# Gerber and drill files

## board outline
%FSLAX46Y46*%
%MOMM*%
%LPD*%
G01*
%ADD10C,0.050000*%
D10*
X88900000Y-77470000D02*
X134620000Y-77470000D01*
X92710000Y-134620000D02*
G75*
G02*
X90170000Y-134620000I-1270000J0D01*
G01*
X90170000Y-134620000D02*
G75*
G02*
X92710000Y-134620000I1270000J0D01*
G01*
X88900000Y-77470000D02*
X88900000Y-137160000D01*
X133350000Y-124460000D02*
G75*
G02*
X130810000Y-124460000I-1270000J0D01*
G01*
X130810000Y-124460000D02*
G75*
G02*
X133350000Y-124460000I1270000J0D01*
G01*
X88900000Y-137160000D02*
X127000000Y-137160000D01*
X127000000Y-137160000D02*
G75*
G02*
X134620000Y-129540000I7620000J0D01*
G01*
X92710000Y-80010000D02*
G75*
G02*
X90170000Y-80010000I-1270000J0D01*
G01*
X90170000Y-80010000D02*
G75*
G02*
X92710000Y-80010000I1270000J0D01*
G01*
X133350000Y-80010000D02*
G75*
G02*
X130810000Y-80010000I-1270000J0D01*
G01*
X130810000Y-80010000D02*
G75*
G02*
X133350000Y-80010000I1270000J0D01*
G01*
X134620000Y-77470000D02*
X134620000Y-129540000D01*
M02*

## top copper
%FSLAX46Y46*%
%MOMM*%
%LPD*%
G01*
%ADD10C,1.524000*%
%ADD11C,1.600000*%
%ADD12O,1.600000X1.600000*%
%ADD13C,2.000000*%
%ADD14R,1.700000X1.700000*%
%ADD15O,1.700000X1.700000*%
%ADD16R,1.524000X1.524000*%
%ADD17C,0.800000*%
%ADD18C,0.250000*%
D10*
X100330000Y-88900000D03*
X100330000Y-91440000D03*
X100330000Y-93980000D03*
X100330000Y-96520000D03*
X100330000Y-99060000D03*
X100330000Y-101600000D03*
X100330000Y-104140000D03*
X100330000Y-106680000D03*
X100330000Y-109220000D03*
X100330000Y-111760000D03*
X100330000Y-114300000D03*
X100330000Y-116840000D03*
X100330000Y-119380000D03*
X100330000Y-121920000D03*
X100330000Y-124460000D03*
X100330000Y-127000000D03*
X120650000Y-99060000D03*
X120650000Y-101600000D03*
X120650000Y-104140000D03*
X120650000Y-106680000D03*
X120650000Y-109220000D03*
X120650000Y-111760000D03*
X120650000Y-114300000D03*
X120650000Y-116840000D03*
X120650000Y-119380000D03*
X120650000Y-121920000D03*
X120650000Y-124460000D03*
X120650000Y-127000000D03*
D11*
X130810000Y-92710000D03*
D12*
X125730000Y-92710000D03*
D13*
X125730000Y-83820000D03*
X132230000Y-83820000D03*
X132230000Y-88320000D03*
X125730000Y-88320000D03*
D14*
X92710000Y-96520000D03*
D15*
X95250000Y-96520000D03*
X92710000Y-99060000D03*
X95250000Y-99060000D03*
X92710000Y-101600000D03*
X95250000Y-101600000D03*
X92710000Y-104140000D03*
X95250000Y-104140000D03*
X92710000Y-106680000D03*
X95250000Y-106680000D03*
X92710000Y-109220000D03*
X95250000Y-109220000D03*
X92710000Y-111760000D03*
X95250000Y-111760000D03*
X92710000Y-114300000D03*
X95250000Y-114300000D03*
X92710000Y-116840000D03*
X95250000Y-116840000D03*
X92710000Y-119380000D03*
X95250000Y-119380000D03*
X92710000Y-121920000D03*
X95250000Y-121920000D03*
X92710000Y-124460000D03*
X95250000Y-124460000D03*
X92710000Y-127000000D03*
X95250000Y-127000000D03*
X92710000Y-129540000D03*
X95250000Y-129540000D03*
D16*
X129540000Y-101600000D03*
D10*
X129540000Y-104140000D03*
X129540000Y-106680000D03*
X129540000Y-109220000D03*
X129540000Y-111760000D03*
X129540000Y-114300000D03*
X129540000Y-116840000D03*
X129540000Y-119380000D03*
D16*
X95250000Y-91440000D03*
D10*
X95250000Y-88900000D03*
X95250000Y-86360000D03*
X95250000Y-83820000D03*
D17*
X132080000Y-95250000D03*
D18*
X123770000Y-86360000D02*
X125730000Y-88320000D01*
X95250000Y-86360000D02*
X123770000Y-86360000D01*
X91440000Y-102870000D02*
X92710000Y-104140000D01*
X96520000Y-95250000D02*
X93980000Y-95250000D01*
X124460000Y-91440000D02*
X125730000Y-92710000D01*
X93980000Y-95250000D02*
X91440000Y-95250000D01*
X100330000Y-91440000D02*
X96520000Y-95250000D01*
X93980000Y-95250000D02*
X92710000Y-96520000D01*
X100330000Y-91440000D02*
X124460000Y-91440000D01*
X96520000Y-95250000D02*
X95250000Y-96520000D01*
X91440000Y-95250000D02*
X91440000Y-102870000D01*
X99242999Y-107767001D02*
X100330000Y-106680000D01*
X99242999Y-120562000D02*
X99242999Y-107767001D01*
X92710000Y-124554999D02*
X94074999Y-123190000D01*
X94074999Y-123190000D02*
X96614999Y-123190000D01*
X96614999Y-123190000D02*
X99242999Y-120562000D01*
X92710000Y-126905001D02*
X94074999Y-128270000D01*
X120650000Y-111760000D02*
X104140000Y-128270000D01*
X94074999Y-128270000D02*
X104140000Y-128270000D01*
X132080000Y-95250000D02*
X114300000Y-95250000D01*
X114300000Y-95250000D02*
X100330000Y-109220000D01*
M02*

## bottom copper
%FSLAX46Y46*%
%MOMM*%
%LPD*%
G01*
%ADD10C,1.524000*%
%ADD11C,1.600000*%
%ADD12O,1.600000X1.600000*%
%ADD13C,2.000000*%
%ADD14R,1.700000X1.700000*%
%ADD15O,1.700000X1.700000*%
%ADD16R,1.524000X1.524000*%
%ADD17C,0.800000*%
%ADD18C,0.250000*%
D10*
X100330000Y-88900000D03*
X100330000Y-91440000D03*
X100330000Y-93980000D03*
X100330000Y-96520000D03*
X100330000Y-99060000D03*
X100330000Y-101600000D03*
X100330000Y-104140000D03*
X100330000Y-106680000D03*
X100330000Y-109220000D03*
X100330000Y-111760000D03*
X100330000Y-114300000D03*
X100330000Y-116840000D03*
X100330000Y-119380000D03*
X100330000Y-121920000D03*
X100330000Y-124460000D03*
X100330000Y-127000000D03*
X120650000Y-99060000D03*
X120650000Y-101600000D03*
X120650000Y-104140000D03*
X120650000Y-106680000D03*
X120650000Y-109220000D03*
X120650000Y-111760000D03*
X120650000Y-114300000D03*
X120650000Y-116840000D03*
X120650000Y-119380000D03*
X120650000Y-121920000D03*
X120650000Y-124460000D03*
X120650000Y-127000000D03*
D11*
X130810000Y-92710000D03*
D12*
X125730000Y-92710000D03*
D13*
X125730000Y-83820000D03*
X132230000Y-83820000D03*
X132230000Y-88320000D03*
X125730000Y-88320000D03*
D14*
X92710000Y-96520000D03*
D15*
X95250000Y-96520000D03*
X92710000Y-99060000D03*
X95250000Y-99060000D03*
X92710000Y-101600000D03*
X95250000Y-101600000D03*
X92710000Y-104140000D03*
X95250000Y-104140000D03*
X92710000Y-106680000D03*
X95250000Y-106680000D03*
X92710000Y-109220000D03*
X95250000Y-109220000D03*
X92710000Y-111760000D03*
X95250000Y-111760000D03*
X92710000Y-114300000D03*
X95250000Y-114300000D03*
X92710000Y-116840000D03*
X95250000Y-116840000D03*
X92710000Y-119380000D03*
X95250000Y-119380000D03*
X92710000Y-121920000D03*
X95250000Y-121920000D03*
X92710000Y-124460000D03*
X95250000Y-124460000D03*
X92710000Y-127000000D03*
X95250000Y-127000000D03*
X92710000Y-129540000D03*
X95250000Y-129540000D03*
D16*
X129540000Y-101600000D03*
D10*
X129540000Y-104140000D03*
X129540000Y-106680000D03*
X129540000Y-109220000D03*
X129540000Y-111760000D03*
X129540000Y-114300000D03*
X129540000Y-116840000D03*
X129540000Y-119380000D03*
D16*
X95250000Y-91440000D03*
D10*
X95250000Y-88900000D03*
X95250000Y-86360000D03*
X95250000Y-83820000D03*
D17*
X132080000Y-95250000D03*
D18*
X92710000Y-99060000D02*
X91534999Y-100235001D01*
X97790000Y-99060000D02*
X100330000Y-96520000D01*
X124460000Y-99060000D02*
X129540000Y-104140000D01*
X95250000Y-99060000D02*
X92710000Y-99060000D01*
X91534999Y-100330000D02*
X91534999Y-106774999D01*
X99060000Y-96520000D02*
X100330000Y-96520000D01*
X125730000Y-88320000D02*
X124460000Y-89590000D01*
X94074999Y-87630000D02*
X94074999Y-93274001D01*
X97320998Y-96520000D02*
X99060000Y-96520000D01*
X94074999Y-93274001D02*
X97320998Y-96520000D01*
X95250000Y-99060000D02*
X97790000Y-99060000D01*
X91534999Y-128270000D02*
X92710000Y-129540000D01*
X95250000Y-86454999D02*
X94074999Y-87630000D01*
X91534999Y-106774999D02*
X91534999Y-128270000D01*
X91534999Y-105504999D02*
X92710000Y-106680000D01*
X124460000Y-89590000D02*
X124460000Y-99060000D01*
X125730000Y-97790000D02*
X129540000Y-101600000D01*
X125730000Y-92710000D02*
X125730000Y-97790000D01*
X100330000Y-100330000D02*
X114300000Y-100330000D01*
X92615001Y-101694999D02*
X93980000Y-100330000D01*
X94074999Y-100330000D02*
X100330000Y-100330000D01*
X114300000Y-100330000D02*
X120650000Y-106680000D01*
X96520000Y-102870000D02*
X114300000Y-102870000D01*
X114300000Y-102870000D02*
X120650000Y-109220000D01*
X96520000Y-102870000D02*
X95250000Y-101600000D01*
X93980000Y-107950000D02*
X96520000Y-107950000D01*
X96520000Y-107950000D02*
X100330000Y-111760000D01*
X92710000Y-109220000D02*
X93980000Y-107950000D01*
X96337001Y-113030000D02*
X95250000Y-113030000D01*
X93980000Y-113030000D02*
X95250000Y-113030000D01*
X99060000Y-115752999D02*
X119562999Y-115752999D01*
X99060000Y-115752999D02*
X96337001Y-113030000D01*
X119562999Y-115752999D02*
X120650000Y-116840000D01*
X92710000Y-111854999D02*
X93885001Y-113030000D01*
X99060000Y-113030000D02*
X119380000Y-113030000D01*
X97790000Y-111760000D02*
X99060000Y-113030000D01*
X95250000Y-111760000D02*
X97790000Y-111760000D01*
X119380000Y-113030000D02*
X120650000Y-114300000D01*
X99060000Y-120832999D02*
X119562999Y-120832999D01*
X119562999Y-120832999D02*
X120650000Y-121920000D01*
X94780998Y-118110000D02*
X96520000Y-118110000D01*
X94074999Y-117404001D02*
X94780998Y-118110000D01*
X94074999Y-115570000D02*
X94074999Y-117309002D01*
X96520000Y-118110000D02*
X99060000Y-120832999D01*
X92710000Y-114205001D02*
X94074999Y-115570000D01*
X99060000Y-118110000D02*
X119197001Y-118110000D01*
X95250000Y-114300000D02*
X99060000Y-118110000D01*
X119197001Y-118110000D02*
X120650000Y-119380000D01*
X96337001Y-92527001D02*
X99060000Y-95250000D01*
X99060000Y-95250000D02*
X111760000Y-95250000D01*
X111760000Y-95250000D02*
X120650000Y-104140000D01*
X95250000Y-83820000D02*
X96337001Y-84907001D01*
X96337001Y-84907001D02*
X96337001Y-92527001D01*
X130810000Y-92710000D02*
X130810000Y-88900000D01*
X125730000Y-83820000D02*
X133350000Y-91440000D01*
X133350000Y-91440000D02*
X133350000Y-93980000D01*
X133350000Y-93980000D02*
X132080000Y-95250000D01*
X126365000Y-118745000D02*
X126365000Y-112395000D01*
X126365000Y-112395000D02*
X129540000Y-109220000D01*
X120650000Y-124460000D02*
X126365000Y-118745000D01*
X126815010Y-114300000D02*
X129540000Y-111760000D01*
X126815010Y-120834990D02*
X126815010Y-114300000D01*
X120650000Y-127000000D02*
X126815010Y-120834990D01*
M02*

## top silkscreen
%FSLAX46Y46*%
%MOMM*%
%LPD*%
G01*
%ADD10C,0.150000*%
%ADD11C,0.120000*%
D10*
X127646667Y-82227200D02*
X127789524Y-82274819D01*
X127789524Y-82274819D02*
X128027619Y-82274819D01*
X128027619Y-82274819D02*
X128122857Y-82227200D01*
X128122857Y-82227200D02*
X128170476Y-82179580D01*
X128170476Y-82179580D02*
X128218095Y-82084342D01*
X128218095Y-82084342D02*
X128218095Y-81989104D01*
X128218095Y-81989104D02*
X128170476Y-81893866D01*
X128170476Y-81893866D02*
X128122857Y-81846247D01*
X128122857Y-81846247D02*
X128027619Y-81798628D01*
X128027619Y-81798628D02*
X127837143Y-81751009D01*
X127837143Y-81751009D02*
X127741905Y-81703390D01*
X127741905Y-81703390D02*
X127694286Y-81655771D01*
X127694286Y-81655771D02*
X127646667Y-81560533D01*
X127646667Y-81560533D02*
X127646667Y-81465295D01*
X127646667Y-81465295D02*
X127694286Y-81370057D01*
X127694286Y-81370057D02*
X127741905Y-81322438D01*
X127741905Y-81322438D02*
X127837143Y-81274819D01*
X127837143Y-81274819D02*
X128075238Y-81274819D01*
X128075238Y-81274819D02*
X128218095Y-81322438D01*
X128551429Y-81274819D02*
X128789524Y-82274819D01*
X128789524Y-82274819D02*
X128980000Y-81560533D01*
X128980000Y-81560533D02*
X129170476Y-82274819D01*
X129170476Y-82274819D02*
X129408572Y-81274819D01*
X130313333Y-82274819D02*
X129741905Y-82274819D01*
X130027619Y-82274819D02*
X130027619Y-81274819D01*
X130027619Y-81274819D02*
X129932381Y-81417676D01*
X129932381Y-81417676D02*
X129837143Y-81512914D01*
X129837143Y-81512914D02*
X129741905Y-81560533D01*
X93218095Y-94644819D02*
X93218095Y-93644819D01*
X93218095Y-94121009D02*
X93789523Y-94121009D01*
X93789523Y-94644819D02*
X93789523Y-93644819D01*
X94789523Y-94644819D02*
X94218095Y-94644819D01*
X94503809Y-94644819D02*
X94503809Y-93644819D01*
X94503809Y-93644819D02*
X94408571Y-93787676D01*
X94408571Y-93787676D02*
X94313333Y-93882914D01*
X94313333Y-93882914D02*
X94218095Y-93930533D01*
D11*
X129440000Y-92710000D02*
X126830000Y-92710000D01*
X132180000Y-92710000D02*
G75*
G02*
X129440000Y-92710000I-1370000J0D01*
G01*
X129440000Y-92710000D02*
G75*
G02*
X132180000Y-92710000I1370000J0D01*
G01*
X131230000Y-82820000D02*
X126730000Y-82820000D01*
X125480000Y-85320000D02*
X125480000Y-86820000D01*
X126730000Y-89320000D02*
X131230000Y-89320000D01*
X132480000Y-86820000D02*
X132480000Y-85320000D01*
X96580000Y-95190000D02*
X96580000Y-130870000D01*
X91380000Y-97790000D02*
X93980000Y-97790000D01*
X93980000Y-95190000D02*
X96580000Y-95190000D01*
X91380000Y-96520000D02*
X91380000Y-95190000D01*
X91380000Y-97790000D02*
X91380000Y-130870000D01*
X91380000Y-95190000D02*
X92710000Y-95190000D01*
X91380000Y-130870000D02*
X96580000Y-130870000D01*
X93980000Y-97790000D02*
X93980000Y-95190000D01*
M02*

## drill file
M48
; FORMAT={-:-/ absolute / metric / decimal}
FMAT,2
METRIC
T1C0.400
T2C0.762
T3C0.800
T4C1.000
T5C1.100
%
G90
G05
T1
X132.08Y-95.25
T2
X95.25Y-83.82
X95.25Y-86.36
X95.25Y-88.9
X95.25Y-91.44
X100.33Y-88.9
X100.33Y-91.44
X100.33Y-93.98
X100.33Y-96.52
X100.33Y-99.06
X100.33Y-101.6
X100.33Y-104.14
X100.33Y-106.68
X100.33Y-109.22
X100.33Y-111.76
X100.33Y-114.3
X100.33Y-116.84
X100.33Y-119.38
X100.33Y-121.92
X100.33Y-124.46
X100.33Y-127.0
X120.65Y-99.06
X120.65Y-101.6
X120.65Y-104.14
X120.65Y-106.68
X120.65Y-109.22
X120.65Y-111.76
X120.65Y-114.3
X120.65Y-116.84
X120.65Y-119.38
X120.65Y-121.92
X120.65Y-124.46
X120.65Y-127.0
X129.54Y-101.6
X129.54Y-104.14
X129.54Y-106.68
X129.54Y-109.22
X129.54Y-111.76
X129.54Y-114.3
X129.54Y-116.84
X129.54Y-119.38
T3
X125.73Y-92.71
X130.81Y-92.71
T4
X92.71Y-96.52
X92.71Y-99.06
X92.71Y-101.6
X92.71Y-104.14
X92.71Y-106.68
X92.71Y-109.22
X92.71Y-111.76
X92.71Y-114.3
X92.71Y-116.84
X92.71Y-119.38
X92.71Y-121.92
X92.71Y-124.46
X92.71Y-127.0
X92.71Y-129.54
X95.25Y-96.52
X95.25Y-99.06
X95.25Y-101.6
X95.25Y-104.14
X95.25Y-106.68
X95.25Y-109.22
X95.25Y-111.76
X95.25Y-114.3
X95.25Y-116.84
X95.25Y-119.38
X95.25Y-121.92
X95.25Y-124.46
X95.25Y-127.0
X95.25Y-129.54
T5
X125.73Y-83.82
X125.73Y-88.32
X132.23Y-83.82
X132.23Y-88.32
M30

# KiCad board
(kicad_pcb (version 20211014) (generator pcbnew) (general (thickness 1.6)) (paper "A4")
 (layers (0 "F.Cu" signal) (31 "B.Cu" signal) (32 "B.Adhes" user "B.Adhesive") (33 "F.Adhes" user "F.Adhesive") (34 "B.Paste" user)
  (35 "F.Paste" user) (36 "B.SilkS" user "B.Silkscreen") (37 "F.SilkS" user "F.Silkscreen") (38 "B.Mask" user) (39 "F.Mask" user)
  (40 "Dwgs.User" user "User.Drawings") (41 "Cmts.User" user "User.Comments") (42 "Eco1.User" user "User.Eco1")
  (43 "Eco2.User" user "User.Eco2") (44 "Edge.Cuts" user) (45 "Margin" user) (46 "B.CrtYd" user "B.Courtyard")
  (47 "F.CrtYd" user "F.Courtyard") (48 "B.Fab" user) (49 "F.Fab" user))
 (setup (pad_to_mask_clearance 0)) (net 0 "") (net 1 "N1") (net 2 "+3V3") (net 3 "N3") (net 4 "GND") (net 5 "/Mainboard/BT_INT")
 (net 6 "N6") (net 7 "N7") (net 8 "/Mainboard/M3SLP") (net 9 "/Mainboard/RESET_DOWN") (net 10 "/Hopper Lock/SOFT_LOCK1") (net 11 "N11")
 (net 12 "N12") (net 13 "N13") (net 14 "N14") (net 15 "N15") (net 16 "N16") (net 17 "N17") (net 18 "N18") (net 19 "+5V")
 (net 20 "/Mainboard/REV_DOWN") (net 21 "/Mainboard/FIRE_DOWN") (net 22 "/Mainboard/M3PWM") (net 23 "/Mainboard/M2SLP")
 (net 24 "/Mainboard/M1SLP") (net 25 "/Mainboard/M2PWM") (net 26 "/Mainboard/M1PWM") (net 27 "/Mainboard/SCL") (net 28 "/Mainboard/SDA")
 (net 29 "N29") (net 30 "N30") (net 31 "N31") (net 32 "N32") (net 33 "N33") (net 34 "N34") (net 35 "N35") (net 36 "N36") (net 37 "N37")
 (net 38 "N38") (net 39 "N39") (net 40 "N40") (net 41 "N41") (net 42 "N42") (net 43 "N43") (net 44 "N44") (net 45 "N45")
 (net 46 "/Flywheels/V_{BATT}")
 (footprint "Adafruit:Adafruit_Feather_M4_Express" (layer "F.Cu") (at 110.49 107.95)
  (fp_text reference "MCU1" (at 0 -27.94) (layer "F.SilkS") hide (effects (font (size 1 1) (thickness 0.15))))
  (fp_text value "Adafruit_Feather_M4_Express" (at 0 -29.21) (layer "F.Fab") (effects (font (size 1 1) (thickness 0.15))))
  (pad "1" thru_hole circle locked (at -10.16 -19.05) (size 1.524 1.524) (drill 0.762) (layers *.Cu *.Mask) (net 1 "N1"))
  (pad "2" thru_hole circle locked (at -10.16 -16.51) (size 1.524 1.524) (drill 0.762) (layers *.Cu *.Mask) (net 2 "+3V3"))
  (pad "3" thru_hole circle locked (at -10.16 -13.97) (size 1.524 1.524) (drill 0.762) (layers *.Cu *.Mask) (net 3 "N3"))
  (pad "4" thru_hole circle locked (at -10.16 -11.43) (size 1.524 1.524) (drill 0.762) (layers *.Cu *.Mask) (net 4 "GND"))
  (pad "5" thru_hole circle locked (at -10.16 -8.89) (size 1.524 1.524) (drill 0.762) (layers *.Cu *.Mask) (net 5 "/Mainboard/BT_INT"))
  (pad "6" thru_hole circle locked (at -10.16 -6.35) (size 1.524 1.524) (drill 0.762) (layers *.Cu *.Mask) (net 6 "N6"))
  (pad "7" thru_hole circle locked (at -10.16 -3.81) (size 1.524 1.524) (drill 0.762) (layers *.Cu *.Mask) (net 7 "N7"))
  (pad "8" thru_hole circle locked (at -10.16 -1.27) (size 1.524 1.524) (drill 0.762) (layers *.Cu *.Mask) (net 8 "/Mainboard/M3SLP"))
  (pad "9" thru_hole circle locked (at -10.16 1.27) (size 1.524 1.524) (drill 0.762) (layers *.Cu *.Mask) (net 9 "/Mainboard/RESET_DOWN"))
  (pad "10" thru_hole circle locked (at -10.16 3.81) (size 1.524 1.524) (drill 0.762) (layers *.Cu *.Mask)
   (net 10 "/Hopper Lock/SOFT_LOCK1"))
  (pad "11" thru_hole circle locked (at -10.16 6.35) (size 1.524 1.524) (drill 0.762) (layers *.Cu *.Mask) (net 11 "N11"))
  (pad "12" thru_hole circle locked (at -10.16 8.89) (size 1.524 1.524) (drill 0.762) (layers *.Cu *.Mask) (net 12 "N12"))
  (pad "13" thru_hole circle locked (at -10.16 11.43) (size 1.524 1.524) (drill 0.762) (layers *.Cu *.Mask) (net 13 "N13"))
  (pad "14" thru_hole circle locked (at -10.16 13.97) (size 1.524 1.524) (drill 0.762) (layers *.Cu *.Mask) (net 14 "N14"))
  (pad "15" thru_hole circle locked (at -10.16 16.51) (size 1.524 1.524) (drill 0.762) (layers *.Cu *.Mask) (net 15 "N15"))
  (pad "16" thru_hole circle locked (at -10.16 19.05) (size 1.524 1.524) (drill 0.762) (layers *.Cu *.Mask) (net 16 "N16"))
  (pad "17" thru_hole circle locked (at 10.16 -8.89) (size 1.524 1.524) (drill 0.762) (layers *.Cu *.Mask) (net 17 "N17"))
  (pad "18" thru_hole circle locked (at 10.16 -6.35) (size 1.524 1.524) (drill 0.762) (layers *.Cu *.Mask) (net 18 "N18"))
  (pad "19" thru_hole circle locked (at 10.16 -3.81) (size 1.524 1.524) (drill 0.762) (layers *.Cu *.Mask) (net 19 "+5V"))
  (pad "20" thru_hole circle locked (at 10.16 -1.27) (size 1.524 1.524) (drill 0.762) (layers *.Cu *.Mask) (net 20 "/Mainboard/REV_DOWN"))
  (pad "21" thru_hole circle locked (at 10.16 1.27) (size 1.524 1.524) (drill 0.762) (layers *.Cu *.Mask) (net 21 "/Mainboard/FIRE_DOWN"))
  (pad "22" thru_hole circle locked (at 10.16 3.81) (size 1.524 1.524) (drill 0.762) (layers *.Cu *.Mask) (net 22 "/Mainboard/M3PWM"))
  (pad "23" thru_hole circle locked (at 10.16 6.35) (size 1.524 1.524) (drill 0.762) (layers *.Cu *.Mask) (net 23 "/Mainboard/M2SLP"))
  (pad "24" thru_hole circle locked (at 10.16 8.89) (size 1.524 1.524) (drill 0.762) (layers *.Cu *.Mask) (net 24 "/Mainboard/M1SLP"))
  (pad "25" thru_hole circle locked (at 10.16 11.43) (size 1.524 1.524) (drill 0.762) (layers *.Cu *.Mask) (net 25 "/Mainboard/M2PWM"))
  (pad "26" thru_hole circle locked (at 10.16 13.97) (size 1.524 1.524) (drill 0.762) (layers *.Cu *.Mask) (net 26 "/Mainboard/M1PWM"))
  (pad "27" thru_hole circle locked (at 10.16 16.51) (size 1.524 1.524) (drill 0.762) (layers *.Cu *.Mask) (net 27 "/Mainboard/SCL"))
  (pad "28" thru_hole circle locked (at 10.16 19.05) (size 1.524 1.524) (drill 0.762) (layers *.Cu *.Mask) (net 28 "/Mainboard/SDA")))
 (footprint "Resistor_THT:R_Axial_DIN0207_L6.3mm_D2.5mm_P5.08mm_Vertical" (layer "F.Cu") (at 130.81 92.71 180)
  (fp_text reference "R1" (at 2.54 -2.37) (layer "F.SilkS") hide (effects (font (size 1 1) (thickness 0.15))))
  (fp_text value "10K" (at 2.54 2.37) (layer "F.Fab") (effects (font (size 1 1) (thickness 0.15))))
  (fp_line (start 1.37 0) (end 3.98 0) (layer "F.SilkS") (width 0.12))
  (fp_circle (center 0 0) (end 1.37 0) (layer "F.SilkS") (width 0.12) (fill none))
  (pad "1" thru_hole circle locked (at 0 0 180) (size 1.6 1.6) (drill 0.8) (layers *.Cu *.Mask) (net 9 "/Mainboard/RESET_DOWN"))
  (pad "2" thru_hole oval locked (at 5.08 0 180) (size 1.6 1.6) (drill 0.8) (layers *.Cu *.Mask) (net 2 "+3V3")))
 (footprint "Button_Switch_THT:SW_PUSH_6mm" (layer "F.Cu") (at 125.73 83.82)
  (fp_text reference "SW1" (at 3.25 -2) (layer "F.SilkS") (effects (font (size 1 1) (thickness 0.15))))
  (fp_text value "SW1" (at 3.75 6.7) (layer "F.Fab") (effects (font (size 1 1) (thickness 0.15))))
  (fp_line (start 5.5 -1) (end 1 -1) (layer "F.SilkS") (width 0.12))
  (fp_line (start -0.25 1.5) (end -0.25 3) (layer "F.SilkS") (width 0.12))
  (fp_line (start 1 5.5) (end 5.5 5.5) (layer "F.SilkS") (width 0.12))
  (fp_line (start 6.75 3) (end 6.75 1.5) (layer "F.SilkS") (width 0.12))
  (pad "1" thru_hole circle locked (at 0 0 90) (size 2 2) (drill 1.1) (layers *.Cu *.Mask) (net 9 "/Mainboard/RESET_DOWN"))
  (pad "1" thru_hole circle locked (at 6.5 0 90) (size 2 2) (drill 1.1) (layers *.Cu *.Mask) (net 9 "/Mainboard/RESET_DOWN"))
  (pad "2" thru_hole circle locked (at 6.5 4.5 90) (size 2 2) (drill 1.1) (layers *.Cu *.Mask) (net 4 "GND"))
  (pad "2" thru_hole circle locked (at 0 4.5 90) (size 2 2) (drill 1.1) (layers *.Cu *.Mask) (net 4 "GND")))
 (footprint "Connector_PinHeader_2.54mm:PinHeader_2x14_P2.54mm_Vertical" (layer "F.Cu") (at 92.71 96.52)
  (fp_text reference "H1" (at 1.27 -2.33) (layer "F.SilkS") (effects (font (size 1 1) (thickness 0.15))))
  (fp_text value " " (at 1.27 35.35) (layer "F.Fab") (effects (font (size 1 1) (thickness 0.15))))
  (fp_line (start 3.87 -1.33) (end 3.87 34.35) (layer "F.SilkS") (width 0.12))
  (fp_line (start -1.33 1.27) (end 1.27 1.27) (layer "F.SilkS") (width 0.12))
  (fp_line (start 1.27 -1.33) (end 3.87 -1.33) (layer "F.SilkS") (width 0.12))
  (fp_line (start -1.33 0) (end -1.33 -1.33) (layer "F.SilkS") (width 0.12))
  (fp_line (start -1.33 1.27) (end -1.33 34.35) (layer "F.SilkS") (width 0.12))
  (fp_line (start -1.33 -1.33) (end 0 -1.33) (layer "F.SilkS") (width 0.12))
  (fp_line (start -1.33 34.35) (end 3.87 34.35) (layer "F.SilkS") (width 0.12))
  (fp_line (start 1.27 1.27) (end 1.27 -1.33) (layer "F.SilkS") (width 0.12))
  (pad "1" thru_hole rect locked (at 0 0) (size 1.7 1.7) (drill 1) (layers *.Cu *.Mask) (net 2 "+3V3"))
  (pad "2" thru_hole oval locked (at 2.54 0) (size 1.7 1.7) (drill 1) (layers *.Cu *.Mask) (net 2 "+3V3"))
  (pad "3" thru_hole oval locked (at 0 2.54) (size 1.7 1.7) (drill 1) (layers *.Cu *.Mask) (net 4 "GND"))
  (pad "4" thru_hole oval locked (at 2.54 2.54) (size 1.7 1.7) (drill 1) (layers *.Cu *.Mask) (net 4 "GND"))
  (pad "5" thru_hole oval locked (at 0 5.08) (size 1.7 1.7) (drill 1) (layers *.Cu *.Mask) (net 20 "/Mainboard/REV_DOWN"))
  (pad "6" thru_hole oval locked (at 2.54 5.08) (size 1.7 1.7) (drill 1) (layers *.Cu *.Mask) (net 21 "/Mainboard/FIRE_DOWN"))
  (pad "7" thru_hole oval locked (at 0 7.62) (size 1.7 1.7) (drill 1) (layers *.Cu *.Mask) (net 2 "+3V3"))
  (pad "8" thru_hole oval locked (at 2.54 7.62) (size 1.7 1.7) (drill 1) (layers *.Cu *.Mask) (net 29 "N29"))
  (pad "9" thru_hole oval locked (at 0 10.16) (size 1.7 1.7) (drill 1) (layers *.Cu *.Mask) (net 4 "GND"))
  (pad "10" thru_hole oval locked (at 2.54 10.16) (size 1.7 1.7) (drill 1) (layers *.Cu *.Mask) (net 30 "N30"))
  (pad "11" thru_hole oval locked (at 0 12.7) (size 1.7 1.7) (drill 1) (layers *.Cu *.Mask) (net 10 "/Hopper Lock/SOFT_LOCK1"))
  (pad "12" thru_hole oval locked (at 2.54 12.7) (size 1.7 1.7) (drill 1) (layers *.Cu *.Mask) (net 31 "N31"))
  (pad "13" thru_hole oval locked (at 0 15.24) (size 1.7 1.7) (drill 1) (layers *.Cu *.Mask) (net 24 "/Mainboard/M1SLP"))
  (pad "14" thru_hole oval locked (at 2.54 15.24) (size 1.7 1.7) (drill 1) (layers *.Cu *.Mask) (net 23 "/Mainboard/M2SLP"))
  (pad "15" thru_hole oval locked (at 0 17.78) (size 1.7 1.7) (drill 1) (layers *.Cu *.Mask) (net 26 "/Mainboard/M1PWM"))
  (pad "16" thru_hole oval locked (at 2.54 17.78) (size 1.7 1.7) (drill 1) (layers *.Cu *.Mask) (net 25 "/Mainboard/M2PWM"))
  (pad "17" thru_hole oval locked (at 0 20.32) (size 1.7 1.7) (drill 1) (layers *.Cu *.Mask) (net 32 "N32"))
  (pad "18" thru_hole oval locked (at 2.54 20.32) (size 1.7 1.7) (drill 1) (layers *.Cu *.Mask) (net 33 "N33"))
  (pad "19" thru_hole oval locked (at 0 22.86) (size 1.7 1.7) (drill 1) (layers *.Cu *.Mask) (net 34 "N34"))
  (pad "20" thru_hole oval locked (at 2.54 22.86) (size 1.7 1.7) (drill 1) (layers *.Cu *.Mask) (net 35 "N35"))
  (pad "21" thru_hole oval locked (at 0 25.4) (size 1.7 1.7) (drill 1) (layers *.Cu *.Mask) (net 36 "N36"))
  (pad "22" thru_hole oval locked (at 2.54 25.4) (size 1.7 1.7) (drill 1) (layers *.Cu *.Mask) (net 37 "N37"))
  (pad "23" thru_hole oval locked (at 0 27.94) (size 1.7 1.7) (drill 1) (layers *.Cu *.Mask) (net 8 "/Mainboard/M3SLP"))
  (pad "24" thru_hole oval locked (at 2.54 27.94) (size 1.7 1.7) (drill 1) (layers *.Cu *.Mask) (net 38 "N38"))
  (pad "25" thru_hole oval locked (at 0 30.48) (size 1.7 1.7) (drill 1) (layers *.Cu *.Mask) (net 22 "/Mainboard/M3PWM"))
  (pad "26" thru_hole oval locked (at 2.54 30.48) (size 1.7 1.7) (drill 1) (layers *.Cu *.Mask) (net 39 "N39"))
  (pad "27" thru_hole oval locked (at 0 33.02) (size 1.7 1.7) (drill 1) (layers *.Cu *.Mask) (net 4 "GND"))
  (pad "28" thru_hole oval locked (at 2.54 33.02) (size 1.7 1.7) (drill 1) (layers *.Cu *.Mask) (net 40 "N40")))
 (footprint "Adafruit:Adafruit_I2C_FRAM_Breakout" (layer "B.Cu") (at 124.46 110.49 -90)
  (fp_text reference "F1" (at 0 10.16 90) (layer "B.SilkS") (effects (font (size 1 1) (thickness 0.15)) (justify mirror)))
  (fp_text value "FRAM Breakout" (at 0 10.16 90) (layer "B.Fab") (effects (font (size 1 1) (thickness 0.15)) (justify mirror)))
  (pad "1" thru_hole rect locked (at -8.89 -5.08 270) (size 1.524 1.524) (drill 0.762) (layers *.Cu *.Mask) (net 2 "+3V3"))
  (pad "2" thru_hole circle locked (at -6.35 -5.08 270) (size 1.524 1.524) (drill 0.762) (layers *.Cu *.Mask) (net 4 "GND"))
  (pad "3" thru_hole circle locked (at -3.81 -5.08 270) (size 1.524 1.524) (drill 0.762) (layers *.Cu *.Mask) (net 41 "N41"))
  (pad "4" thru_hole circle locked (at -1.27 -5.08 270) (size 1.524 1.524) (drill 0.762) (layers *.Cu *.Mask) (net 27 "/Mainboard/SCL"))
  (pad "5" thru_hole circle locked (at 1.27 -5.08 270) (size 1.524 1.524) (drill 0.762) (layers *.Cu *.Mask) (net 28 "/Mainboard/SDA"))
  (pad "6" thru_hole circle locked (at 3.81 -5.08 270) (size 1.524 1.524) (drill 0.762) (layers *.Cu *.Mask) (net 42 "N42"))
  (pad "7" thru_hole circle locked (at 6.35 -5.08 270) (size 1.524 1.524) (drill 0.762) (layers *.Cu *.Mask) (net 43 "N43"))
  (pad "8" thru_hole circle locked (at 8.89 -5.08 270) (size 1.524 1.524) (drill 0.762) (layers *.Cu *.Mask) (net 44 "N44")))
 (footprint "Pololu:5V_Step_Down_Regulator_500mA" (layer "B.Cu") (at 100.33 87.63 90)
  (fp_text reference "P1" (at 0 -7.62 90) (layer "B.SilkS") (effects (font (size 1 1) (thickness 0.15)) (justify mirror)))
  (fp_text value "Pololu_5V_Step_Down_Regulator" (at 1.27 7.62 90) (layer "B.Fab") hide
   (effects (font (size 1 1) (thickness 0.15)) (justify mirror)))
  (pad "1" thru_hole rect locked (at -3.81 -5.08 90) (size 1.524 1.524) (drill 0.762) (layers *.Cu *.Mask) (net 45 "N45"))
  (pad "2" thru_hole circle locked (at -1.27 -5.08 90) (size 1.524 1.524) (drill 0.762) (layers *.Cu *.Mask) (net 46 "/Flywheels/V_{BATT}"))
  (pad "3" thru_hole circle locked (at 1.27 -5.08 90) (size 1.524 1.524) (drill 0.762) (layers *.Cu *.Mask) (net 4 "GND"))
  (pad "4" thru_hole circle locked (at 3.81 -5.08 90) (size 1.524 1.524) (drill 0.762) (layers *.Cu *.Mask) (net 19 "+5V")))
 (gr_line (start 88.9 77.47) (end 134.62 77.47) (layer "Edge.Cuts") (width 0.05))
 (gr_circle (center 91.44 134.62) (end 91.44 135.89) (layer "Edge.Cuts") (width 0.05) (fill none))
 (gr_line (start 88.9 77.47) (end 88.9 137.16) (layer "Edge.Cuts") (width 0.05))
 (gr_circle (center 132.08 124.46) (end 133.35 124.46) (layer "Edge.Cuts") (width 0.05) (fill none))
 (gr_line (start 88.9 137.16) (end 127 137.16) (layer "Edge.Cuts") (width 0.05))
 (gr_arc (start 127 137.16) (mid 129.231846 131.771846) (end 134.62 129.54) (layer "Edge.Cuts") (width 0.05))
 (gr_circle (center 91.44 80.01) (end 90.17 80.01) (layer "Edge.Cuts") (width 0.05) (fill none))
 (gr_circle (center 132.08 80.01) (end 133.35 80.01) (layer "Edge.Cuts") (width 0.05) (fill none))
 (gr_line (start 134.62 77.47) (end 134.62 129.54) (layer "Edge.Cuts") (width 0.05))
 (segment (start 123.77 86.36) (end 125.73 88.32) (width 0.25) (layer "F.Cu") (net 4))
 (segment (start 95.25 86.36) (end 123.77 86.36) (width 0.25) (layer "F.Cu") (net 4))
 (segment (start 92.71 99.06) (end 91.534999 100.235001) (width 0.25) (layer "B.Cu") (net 4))
 (segment (start 97.79 99.06) (end 100.33 96.52) (width 0.25) (layer "B.Cu") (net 4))
 (segment (start 124.46 99.06) (end 129.54 104.14) (width 0.25) (layer "B.Cu") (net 4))
 (segment (start 95.25 99.06) (end 92.71 99.06) (width 0.25) (layer "B.Cu") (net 4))
 (segment (start 91.534999 100.33) (end 91.534999 106.774999) (width 0.25) (layer "B.Cu") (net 4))
 (segment (start 99.06 96.52) (end 100.33 96.52) (width 0.25) (layer "B.Cu") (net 4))
 (segment (start 125.73 88.32) (end 124.46 89.59) (width 0.25) (layer "B.Cu") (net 4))
 (segment (start 94.074999 87.63) (end 94.074999 93.274001) (width 0.25) (layer "B.Cu") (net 4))
 (segment (start 97.320998 96.52) (end 99.06 96.52) (width 0.25) (layer "B.Cu") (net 4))
 (segment (start 94.074999 93.274001) (end 97.320998 96.52) (width 0.25) (layer "B.Cu") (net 4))
 (segment (start 95.25 99.06) (end 97.79 99.06) (width 0.25) (layer "B.Cu") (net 4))
 (segment (start 91.534999 128.27) (end 92.71 129.54) (width 0.25) (layer "B.Cu") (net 4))
 (segment (start 95.25 86.454999) (end 94.074999 87.63) (width 0.25) (layer "B.Cu") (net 4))
 (segment (start 91.534999 106.774999) (end 91.534999 128.27) (width 0.25) (layer "B.Cu") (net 4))
 (segment (start 91.534999 105.504999) (end 92.71 106.68) (width 0.25) (layer "B.Cu") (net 4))
 (segment (start 124.46 89.59) (end 124.46 99.06) (width 0.25) (layer "B.Cu") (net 4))
 (segment (start 91.44 102.87) (end 92.71 104.14) (width 0.25) (layer "F.Cu") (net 2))
 (segment (start 96.52 95.25) (end 93.98 95.25) (width 0.25) (layer "F.Cu") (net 2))
 (segment (start 124.46 91.44) (end 125.73 92.71) (width 0.25) (layer "F.Cu") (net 2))
 (segment (start 93.98 95.25) (end 91.44 95.25) (width 0.25) (layer "F.Cu") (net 2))
 (segment (start 100.33 91.44) (end 96.52 95.25) (width 0.25) (layer "F.Cu") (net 2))
 (segment (start 93.98 95.25) (end 92.71 96.52) (width 0.25) (layer "F.Cu") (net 2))
 (segment (start 100.33 91.44) (end 124.46 91.44) (width 0.25) (layer "F.Cu") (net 2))
 (segment (start 96.52 95.25) (end 95.25 96.52) (width 0.25) (layer "F.Cu") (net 2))
 (segment (start 91.44 95.25) (end 91.44 102.87) (width 0.25) (layer "F.Cu") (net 2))
 (segment (start 125.73 97.79) (end 129.54 101.6) (width 0.25) (layer "B.Cu") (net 2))
 (segment (start 125.73 92.71) (end 125.73 97.79) (width 0.25) (layer "B.Cu") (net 2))
 (segment (start 100.33 100.33) (end 114.3 100.33) (width 0.25) (layer "B.Cu") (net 20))
 (segment (start 92.615001 101.694999) (end 93.98 100.33) (width 0.25) (layer "B.Cu") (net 20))
 (segment (start 94.074999 100.33) (end 100.33 100.33) (width 0.25) (layer "B.Cu") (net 20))
 (segment (start 114.3 100.33) (end 120.65 106.68) (width 0.25) (layer "B.Cu") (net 20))
 (segment (start 96.52 102.87) (end 114.3 102.87) (width 0.25) (layer "B.Cu") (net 21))
 (segment (start 114.3 102.87) (end 120.65 109.22) (width 0.25) (layer "B.Cu") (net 21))
 (segment (start 96.52 102.87) (end 95.25 101.6) (width 0.25) (layer "B.Cu") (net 21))
 (segment (start 93.98 107.95) (end 96.52 107.95) (width 0.25) (layer "B.Cu") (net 10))
 (segment (start 96.52 107.95) (end 100.33 111.76) (width 0.25) (layer "B.Cu") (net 10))
 (segment (start 92.71 109.22) (end 93.98 107.95) (width 0.25) (layer "B.Cu") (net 10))
 (segment (start 96.337001 113.03) (end 95.25 113.03) (width 0.25) (layer "B.Cu") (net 24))
 (segment (start 93.98 113.03) (end 95.25 113.03) (width 0.25) (layer "B.Cu") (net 24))
 (segment (start 99.06 115.752999) (end 119.562999 115.752999) (width 0.25) (layer "B.Cu") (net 24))
 (segment (start 99.06 115.752999) (end 96.337001 113.03) (width 0.25) (layer "B.Cu") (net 24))
 (segment (start 119.562999 115.752999) (end 120.65 116.84) (width 0.25) (layer "B.Cu") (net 24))
 (segment (start 92.71 111.854999) (end 93.885001 113.03) (width 0.25) (layer "B.Cu") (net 24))
 (segment (start 99.06 113.03) (end 119.38 113.03) (width 0.25) (layer "B.Cu") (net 23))
 (segment (start 97.79 111.76) (end 99.06 113.03) (width 0.25) (layer "B.Cu") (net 23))
 (segment (start 95.25 111.76) (end 97.79 111.76) (width 0.25) (layer "B.Cu") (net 23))
 (segment (start 119.38 113.03) (end 120.65 114.3) (width 0.25) (layer "B.Cu") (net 23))
 (segment (start 99.06 120.832999) (end 119.562999 120.832999) (width 0.25) (layer "B.Cu") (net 26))
 (segment (start 119.562999 120.832999) (end 120.65 121.92) (width 0.25) (layer "B.Cu") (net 26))
 (segment (start 94.780998 118.11) (end 96.52 118.11) (width 0.25) (layer "B.Cu") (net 26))
 (segment (start 94.074999 117.404001) (end 94.780998 118.11) (width 0.25) (layer "B.Cu") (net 26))
 (segment (start 94.074999 115.57) (end 94.074999 117.309002) (width 0.25) (layer "B.Cu") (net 26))
 (segment (start 96.52 118.11) (end 99.06 120.832999) (width 0.25) (layer "B.Cu") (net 26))
 (segment (start 92.71 114.205001) (end 94.074999 115.57) (width 0.25) (layer "B.Cu") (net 26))
 (segment (start 99.06 118.11) (end 119.197001 118.11) (width 0.25) (layer "B.Cu") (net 25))
 (segment (start 95.25 114.3) (end 99.06 118.11) (width 0.25) (layer "B.Cu") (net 25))
 (segment (start 119.197001 118.11) (end 120.65 119.38) (width 0.25) (layer "B.Cu") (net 25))
 (segment (start 99.242999 107.767001) (end 100.33 106.68) (width 0.25) (layer "F.Cu") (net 8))
 (segment (start 99.242999 120.562) (end 99.242999 107.767001) (width 0.25) (layer "F.Cu") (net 8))
 (segment (start 92.71 124.554999) (end 94.074999 123.19) (width 0.25) (layer "F.Cu") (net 8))
 (segment (start 94.074999 123.19) (end 96.614999 123.19) (width 0.25) (layer "F.Cu") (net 8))
 (segment (start 96.614999 123.19) (end 99.242999 120.562) (width 0.25) (layer "F.Cu") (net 8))
 (segment (start 92.71 126.905001) (end 94.074999 128.27) (width 0.25) (layer "F.Cu") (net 22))
 (segment (start 120.65 111.76) (end 104.14 128.27) (width 0.25) (layer "F.Cu") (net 22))
 (segment (start 94.074999 128.27) (end 104.14 128.27) (width 0.25) (layer "F.Cu") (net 22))
 (segment (start 96.337001 92.527001) (end 99.06 95.25) (width 0.25) (layer "B.Cu") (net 19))
 (segment (start 99.06 95.25) (end 111.76 95.25) (width 0.25) (layer "B.Cu") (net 19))
 (segment (start 111.76 95.25) (end 120.65 104.14) (width 0.25) (layer "B.Cu") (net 19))
 (segment (start 95.25 83.82) (end 96.337001 84.907001) (width 0.25) (layer "B.Cu") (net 19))
 (segment (start 96.337001 84.907001) (end 96.337001 92.527001) (width 0.25) (layer "B.Cu") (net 19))
 (segment (start 132.08 95.25) (end 114.3 95.25) (width 0.25) (layer "F.Cu") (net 9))
 (segment (start 114.3 95.25) (end 100.33 109.22) (width 0.25) (layer "F.Cu") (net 9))
 (via (at 132.08 95.25) (size 0.8) (drill 0.4) (layers "F.Cu" "B.Cu") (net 9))
 (segment (start 130.81 92.71) (end 130.81 88.9) (width 0.25) (layer "B.Cu") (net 9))
 (segment (start 125.73 83.82) (end 133.35 91.44) (width 0.25) (layer "B.Cu") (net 9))
 (segment (start 133.35 91.44) (end 133.35 93.98) (width 0.25) (layer "B.Cu") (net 9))
 (segment (start 133.35 93.98) (end 132.08 95.25) (width 0.25) (layer "B.Cu") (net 9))
 (segment (start 126.365 118.745) (end 126.365 112.395) (width 0.25) (layer "B.Cu") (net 27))
 (segment (start 126.365 112.395) (end 129.54 109.22) (width 0.25) (layer "B.Cu") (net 27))
 (segment (start 120.65 124.46) (end 126.365 118.745) (width 0.25) (layer "B.Cu") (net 27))
 (segment (start 126.81501 114.3) (end 129.54 111.76) (width 0.25) (layer "B.Cu") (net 28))
 (segment (start 126.81501 120.83499) (end 126.81501 114.3) (width 0.25) (layer "B.Cu") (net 28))
 (segment (start 120.65 127) (end 126.81501 120.83499) (width 0.25) (layer "B.Cu") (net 28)))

